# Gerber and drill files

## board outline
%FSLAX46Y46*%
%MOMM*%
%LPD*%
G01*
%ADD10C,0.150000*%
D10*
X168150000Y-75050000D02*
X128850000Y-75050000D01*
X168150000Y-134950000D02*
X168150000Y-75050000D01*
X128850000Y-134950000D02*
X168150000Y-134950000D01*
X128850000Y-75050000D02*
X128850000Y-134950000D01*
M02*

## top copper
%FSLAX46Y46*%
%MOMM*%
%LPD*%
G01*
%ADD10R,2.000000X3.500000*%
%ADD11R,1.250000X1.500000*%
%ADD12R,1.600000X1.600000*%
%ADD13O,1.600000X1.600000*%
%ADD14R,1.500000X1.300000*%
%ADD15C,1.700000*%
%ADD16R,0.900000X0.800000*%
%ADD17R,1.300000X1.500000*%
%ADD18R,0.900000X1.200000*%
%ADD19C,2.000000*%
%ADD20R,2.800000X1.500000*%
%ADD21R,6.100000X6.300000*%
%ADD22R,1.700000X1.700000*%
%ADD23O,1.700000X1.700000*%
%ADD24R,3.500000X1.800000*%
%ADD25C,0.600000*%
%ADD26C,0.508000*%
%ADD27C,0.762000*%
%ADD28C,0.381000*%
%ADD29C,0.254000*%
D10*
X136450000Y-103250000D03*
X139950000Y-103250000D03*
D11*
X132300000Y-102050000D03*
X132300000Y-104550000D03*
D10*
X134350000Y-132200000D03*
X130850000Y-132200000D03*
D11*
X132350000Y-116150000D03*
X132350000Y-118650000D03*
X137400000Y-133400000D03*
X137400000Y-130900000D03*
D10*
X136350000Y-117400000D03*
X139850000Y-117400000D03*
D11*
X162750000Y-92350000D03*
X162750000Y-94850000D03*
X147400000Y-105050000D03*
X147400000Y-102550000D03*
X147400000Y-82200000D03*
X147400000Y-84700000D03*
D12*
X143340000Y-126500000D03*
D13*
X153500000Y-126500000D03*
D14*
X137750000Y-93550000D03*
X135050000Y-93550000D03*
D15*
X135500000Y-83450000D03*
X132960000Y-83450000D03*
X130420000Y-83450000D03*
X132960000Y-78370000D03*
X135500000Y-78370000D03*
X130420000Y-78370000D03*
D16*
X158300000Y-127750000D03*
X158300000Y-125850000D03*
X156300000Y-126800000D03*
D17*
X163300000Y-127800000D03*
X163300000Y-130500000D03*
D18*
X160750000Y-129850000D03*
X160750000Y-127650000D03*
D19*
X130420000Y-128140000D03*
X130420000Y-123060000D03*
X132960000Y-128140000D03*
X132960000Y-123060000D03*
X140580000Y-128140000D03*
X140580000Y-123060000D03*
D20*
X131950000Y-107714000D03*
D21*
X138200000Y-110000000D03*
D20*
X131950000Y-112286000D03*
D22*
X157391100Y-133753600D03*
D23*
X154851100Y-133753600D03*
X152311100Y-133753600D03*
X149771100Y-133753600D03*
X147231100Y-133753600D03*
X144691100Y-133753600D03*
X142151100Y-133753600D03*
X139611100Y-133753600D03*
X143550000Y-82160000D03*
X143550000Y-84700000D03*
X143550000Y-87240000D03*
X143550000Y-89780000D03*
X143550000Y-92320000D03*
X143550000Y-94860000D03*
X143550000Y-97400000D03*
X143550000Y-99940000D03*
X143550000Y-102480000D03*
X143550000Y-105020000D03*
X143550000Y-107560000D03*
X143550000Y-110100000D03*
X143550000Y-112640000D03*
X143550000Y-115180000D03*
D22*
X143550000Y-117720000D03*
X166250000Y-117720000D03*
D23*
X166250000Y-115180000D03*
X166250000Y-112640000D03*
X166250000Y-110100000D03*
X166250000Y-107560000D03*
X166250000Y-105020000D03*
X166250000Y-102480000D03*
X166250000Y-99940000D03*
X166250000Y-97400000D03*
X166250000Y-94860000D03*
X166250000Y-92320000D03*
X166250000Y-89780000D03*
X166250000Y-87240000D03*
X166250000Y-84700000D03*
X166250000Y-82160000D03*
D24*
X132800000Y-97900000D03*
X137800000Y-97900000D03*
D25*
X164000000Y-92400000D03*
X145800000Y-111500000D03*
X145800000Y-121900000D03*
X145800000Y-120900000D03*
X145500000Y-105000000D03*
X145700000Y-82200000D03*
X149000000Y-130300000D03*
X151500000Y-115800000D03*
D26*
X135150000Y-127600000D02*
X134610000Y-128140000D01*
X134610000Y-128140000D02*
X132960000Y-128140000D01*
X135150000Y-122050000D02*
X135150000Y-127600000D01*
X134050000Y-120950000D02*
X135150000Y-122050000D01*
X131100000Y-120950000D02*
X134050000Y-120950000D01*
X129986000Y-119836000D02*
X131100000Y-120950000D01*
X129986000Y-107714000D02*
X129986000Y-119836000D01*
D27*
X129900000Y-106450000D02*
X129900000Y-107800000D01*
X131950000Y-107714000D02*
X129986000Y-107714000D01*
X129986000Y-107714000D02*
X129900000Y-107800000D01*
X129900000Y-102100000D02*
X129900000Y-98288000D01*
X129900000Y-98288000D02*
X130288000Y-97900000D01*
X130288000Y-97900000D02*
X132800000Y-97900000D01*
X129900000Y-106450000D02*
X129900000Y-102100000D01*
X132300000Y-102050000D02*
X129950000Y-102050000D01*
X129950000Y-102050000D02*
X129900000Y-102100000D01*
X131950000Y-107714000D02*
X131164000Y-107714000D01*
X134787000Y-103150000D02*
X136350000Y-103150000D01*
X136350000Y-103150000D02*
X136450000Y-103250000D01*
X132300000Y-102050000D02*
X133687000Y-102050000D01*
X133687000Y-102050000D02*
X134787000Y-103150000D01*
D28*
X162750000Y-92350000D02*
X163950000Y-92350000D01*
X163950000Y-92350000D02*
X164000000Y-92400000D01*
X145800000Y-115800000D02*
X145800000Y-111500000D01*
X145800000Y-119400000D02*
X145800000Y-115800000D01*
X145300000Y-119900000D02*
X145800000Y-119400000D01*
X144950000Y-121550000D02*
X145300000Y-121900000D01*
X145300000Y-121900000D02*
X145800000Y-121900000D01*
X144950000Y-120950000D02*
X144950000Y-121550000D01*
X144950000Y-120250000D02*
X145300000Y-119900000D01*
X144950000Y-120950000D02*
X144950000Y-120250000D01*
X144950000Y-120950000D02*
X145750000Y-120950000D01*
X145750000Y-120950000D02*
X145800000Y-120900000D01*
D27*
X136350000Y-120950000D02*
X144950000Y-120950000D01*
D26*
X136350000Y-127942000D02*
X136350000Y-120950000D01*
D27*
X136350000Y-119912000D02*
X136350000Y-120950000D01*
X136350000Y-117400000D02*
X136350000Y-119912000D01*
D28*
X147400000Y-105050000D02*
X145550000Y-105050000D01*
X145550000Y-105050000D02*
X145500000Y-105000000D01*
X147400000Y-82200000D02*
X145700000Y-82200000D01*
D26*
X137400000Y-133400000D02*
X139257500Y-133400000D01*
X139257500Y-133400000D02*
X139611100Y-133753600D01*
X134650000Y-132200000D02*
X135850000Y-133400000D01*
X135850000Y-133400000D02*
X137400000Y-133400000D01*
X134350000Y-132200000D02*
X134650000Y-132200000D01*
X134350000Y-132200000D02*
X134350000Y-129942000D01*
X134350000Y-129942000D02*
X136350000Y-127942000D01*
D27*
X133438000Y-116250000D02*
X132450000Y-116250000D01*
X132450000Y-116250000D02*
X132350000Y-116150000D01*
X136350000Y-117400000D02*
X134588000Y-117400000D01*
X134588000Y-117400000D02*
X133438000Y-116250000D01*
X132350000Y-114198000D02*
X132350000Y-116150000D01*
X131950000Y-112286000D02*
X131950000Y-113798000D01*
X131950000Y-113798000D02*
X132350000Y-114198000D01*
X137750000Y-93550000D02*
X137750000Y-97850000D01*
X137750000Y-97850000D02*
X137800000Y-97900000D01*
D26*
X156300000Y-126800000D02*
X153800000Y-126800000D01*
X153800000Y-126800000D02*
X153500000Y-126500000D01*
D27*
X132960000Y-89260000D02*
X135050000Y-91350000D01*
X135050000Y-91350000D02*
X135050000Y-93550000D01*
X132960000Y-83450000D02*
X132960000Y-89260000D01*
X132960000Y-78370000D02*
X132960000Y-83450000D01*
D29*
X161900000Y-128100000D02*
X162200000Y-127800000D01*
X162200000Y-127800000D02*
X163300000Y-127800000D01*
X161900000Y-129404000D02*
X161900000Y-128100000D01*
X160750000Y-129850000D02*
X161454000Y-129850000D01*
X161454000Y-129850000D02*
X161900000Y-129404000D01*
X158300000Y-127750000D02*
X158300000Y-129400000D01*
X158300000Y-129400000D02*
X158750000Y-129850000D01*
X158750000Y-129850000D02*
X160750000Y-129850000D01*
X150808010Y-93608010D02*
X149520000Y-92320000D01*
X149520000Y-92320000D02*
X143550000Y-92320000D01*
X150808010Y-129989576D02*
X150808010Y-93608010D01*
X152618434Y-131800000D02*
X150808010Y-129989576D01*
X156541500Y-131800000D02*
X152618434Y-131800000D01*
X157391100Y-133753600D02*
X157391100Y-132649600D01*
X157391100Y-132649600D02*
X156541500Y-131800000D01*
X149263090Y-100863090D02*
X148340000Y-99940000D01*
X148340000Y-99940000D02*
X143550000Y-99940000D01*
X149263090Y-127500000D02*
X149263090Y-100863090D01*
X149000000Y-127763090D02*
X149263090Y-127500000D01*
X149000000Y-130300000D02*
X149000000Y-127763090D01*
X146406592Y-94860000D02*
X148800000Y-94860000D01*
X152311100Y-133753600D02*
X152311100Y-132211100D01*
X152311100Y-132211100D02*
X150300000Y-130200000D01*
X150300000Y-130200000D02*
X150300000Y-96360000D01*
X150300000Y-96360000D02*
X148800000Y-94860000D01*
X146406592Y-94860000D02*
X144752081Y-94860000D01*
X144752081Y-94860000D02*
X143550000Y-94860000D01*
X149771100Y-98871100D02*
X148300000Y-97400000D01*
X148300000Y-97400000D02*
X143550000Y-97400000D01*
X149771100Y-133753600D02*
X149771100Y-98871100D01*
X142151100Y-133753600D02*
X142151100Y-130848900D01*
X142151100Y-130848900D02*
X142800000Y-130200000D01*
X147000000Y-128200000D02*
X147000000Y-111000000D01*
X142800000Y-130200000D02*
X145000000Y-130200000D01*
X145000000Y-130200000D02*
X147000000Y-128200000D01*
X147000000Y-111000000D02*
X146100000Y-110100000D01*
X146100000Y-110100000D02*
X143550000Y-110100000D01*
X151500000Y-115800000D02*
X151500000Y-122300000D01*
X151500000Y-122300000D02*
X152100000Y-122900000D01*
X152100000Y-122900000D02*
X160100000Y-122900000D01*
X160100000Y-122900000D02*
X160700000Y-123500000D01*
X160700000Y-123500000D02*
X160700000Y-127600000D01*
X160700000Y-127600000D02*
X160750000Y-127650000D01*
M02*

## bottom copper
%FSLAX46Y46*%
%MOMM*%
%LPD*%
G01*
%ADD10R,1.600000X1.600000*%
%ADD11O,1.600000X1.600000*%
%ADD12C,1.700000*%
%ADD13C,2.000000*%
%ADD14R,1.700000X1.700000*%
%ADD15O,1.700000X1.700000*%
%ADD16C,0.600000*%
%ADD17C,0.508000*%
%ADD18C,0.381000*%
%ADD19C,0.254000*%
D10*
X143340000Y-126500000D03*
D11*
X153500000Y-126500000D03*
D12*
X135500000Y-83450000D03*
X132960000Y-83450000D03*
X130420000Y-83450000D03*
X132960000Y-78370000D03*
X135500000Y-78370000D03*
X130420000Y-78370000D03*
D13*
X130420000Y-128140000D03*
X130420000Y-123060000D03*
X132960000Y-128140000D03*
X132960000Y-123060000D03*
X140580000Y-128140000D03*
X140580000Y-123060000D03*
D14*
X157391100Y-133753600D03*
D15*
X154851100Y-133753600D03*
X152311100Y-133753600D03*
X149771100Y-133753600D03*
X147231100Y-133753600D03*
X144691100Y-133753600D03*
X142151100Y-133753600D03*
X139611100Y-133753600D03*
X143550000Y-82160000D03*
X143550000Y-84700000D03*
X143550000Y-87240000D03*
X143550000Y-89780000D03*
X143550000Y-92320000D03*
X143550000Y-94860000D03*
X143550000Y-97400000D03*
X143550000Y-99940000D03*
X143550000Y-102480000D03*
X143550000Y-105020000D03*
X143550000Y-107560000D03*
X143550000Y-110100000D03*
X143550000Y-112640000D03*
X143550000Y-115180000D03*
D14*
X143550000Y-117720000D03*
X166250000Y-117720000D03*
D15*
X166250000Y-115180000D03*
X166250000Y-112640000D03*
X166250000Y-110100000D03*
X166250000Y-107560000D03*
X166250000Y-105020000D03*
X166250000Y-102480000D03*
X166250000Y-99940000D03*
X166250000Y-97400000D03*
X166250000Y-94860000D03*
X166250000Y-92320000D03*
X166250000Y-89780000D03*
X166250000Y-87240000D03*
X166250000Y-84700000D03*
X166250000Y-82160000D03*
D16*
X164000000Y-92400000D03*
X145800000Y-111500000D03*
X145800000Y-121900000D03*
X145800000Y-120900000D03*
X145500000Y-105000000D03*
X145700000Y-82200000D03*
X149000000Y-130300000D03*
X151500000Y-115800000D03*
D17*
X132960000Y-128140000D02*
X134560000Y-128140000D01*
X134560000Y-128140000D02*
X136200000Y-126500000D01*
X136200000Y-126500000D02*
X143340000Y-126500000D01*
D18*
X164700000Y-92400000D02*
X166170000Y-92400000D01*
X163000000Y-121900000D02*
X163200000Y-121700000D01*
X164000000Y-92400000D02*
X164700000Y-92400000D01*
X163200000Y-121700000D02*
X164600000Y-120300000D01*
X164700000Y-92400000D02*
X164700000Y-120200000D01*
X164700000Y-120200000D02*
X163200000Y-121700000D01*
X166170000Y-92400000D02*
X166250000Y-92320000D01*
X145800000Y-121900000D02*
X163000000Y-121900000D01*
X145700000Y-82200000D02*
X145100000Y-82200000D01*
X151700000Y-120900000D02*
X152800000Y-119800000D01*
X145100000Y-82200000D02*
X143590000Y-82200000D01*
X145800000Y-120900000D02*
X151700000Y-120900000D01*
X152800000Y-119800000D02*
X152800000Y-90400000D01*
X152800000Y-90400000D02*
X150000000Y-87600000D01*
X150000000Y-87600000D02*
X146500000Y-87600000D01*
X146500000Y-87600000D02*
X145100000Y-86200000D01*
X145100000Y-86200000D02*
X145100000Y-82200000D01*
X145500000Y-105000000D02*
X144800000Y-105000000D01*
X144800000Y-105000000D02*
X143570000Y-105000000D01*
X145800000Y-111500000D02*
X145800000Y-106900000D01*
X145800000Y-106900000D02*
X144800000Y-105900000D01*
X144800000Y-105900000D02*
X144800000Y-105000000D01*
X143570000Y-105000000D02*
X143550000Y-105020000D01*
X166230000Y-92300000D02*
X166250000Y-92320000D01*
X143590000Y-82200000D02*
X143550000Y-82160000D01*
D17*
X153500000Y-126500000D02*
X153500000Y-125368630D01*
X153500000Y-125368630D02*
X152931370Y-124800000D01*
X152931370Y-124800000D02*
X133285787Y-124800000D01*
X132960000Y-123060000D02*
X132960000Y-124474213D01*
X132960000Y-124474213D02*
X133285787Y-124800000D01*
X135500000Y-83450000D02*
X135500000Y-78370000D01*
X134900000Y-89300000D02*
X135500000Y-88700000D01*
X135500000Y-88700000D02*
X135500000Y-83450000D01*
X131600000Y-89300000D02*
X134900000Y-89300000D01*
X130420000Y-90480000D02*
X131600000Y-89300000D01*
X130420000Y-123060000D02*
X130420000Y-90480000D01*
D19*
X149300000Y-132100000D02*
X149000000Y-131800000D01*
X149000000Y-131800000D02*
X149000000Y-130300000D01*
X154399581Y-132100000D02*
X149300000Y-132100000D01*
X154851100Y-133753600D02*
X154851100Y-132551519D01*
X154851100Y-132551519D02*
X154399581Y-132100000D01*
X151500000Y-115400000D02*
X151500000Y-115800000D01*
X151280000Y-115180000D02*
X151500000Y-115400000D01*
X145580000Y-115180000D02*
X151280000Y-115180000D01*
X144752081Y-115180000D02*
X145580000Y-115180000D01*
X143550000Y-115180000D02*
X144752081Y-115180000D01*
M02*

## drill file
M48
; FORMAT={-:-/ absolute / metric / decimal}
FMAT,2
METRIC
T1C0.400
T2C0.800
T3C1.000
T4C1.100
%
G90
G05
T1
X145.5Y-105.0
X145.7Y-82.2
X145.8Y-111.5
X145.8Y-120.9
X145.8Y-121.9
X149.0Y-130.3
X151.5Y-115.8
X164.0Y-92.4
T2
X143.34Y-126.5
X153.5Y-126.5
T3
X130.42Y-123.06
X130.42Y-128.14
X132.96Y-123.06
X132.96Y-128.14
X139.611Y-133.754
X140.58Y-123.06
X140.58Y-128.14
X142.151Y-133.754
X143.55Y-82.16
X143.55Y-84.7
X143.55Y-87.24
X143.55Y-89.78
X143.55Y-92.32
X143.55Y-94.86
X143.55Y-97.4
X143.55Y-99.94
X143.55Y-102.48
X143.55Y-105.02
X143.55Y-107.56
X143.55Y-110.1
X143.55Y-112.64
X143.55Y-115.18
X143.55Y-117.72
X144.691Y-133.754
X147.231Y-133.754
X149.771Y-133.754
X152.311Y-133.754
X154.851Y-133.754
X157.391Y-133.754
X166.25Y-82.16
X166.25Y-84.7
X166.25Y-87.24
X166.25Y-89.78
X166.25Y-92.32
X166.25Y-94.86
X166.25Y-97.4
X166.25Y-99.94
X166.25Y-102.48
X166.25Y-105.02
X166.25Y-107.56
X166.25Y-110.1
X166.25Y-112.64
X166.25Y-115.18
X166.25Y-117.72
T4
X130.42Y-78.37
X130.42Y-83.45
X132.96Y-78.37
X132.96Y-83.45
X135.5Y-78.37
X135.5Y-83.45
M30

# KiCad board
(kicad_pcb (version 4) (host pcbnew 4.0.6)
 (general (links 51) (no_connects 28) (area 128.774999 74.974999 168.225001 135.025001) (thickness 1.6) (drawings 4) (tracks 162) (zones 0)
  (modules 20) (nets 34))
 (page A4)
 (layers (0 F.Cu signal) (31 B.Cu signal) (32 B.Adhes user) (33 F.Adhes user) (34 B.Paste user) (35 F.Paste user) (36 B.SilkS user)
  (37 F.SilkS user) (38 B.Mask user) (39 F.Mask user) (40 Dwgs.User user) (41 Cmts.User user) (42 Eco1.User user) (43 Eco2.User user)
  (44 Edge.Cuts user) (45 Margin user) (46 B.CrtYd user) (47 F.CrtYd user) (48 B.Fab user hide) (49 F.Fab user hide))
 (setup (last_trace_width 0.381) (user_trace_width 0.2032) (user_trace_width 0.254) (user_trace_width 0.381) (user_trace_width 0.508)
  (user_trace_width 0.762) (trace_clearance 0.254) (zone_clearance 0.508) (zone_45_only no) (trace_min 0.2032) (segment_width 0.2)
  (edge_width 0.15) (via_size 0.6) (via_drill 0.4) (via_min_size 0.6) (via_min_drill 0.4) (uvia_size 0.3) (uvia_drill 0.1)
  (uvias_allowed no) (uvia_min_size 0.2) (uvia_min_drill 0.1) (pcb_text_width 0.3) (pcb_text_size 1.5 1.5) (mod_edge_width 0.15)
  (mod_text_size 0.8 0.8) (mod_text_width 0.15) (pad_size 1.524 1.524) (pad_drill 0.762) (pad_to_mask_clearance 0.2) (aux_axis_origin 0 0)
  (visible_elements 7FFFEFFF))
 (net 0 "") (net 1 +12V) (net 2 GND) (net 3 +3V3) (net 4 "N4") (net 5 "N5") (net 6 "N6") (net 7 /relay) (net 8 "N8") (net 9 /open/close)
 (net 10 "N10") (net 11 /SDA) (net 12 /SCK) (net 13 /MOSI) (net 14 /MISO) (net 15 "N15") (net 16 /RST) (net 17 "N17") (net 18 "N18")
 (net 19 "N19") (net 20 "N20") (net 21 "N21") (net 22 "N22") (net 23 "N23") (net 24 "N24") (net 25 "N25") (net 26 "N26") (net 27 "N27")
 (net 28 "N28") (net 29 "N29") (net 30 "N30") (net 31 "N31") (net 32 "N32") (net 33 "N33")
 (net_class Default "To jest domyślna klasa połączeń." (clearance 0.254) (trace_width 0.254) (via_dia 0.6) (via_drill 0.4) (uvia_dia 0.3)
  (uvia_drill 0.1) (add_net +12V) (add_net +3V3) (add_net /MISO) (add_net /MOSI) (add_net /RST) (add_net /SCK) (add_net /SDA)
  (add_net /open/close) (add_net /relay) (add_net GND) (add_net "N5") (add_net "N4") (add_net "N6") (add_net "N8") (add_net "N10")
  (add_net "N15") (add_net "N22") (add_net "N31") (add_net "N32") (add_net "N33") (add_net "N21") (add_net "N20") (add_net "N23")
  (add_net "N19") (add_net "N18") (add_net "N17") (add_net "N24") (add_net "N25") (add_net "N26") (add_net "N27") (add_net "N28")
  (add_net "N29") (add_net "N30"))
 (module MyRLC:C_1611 (layer F.Cu) (at 138.2 103.25 90)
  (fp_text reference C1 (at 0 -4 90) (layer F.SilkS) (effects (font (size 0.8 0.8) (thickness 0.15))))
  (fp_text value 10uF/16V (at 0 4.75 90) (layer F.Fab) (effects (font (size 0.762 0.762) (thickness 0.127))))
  (pad 1 smd rect (at 0 -1.75 90) (size 3.5 2) (layers F.Cu F.Paste F.Mask) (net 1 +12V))
  (pad 2 smd rect (at 0 1.75 90) (size 3.5 2) (layers F.Cu F.Paste F.Mask) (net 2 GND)))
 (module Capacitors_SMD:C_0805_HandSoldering (layer F.Cu) (at 132.3 103.3 270)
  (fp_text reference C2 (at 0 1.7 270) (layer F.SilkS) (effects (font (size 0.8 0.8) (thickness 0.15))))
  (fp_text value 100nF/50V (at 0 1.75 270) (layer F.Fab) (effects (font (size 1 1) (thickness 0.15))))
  (pad 1 smd rect (at -1.25 0 270) (size 1.5 1.25) (layers F.Cu F.Paste F.Mask) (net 1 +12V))
  (pad 2 smd rect (at 1.25 0 270) (size 1.5 1.25) (layers F.Cu F.Paste F.Mask) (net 2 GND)))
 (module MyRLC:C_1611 (layer F.Cu) (at 132.6 132.2 270)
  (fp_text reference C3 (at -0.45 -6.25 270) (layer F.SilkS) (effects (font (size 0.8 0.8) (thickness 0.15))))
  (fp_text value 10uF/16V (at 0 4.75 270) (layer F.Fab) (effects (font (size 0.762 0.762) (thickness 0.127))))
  (pad 1 smd rect (at 0 -1.75 270) (size 3.5 2) (layers F.Cu F.Paste F.Mask) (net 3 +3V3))
  (pad 2 smd rect (at 0 1.75 270) (size 3.5 2) (layers F.Cu F.Paste F.Mask) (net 2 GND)))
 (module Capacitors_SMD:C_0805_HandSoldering (layer F.Cu) (at 132.35 117.4 270)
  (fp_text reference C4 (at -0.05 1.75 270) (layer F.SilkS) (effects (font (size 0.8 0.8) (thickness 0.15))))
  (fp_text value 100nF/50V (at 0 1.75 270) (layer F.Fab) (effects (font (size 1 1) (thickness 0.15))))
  (pad 1 smd rect (at -1.25 0 270) (size 1.5 1.25) (layers F.Cu F.Paste F.Mask) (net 3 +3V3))
  (pad 2 smd rect (at 1.25 0 270) (size 1.5 1.25) (layers F.Cu F.Paste F.Mask) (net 2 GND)))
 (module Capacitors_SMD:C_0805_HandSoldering (layer F.Cu) (at 137.4 132.15 90)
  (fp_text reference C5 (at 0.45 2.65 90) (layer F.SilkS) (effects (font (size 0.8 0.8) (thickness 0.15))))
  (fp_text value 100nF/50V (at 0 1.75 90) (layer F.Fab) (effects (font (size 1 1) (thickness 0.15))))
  (pad 1 smd rect (at -1.25 0 90) (size 1.5 1.25) (layers F.Cu F.Paste F.Mask) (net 3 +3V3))
  (pad 2 smd rect (at 1.25 0 90) (size 1.5 1.25) (layers F.Cu F.Paste F.Mask) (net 2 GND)))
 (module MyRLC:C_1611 (layer F.Cu) (at 138.1 117.4 90)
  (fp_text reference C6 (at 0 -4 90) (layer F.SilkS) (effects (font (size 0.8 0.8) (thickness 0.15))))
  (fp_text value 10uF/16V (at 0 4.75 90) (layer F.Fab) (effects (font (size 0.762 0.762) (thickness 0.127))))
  (pad 1 smd rect (at 0 -1.75 90) (size 3.5 2) (layers F.Cu F.Paste F.Mask) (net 3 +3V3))
  (pad 2 smd rect (at 0 1.75 90) (size 3.5 2) (layers F.Cu F.Paste F.Mask) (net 2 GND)))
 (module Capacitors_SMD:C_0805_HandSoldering (layer F.Cu) (at 162.75 93.6 270)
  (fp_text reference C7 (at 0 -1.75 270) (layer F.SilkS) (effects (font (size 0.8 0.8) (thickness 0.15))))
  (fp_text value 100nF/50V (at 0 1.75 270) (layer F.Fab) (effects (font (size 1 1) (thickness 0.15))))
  (pad 1 smd rect (at -1.25 0 270) (size 1.5 1.25) (layers F.Cu F.Paste F.Mask) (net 3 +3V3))
  (pad 2 smd rect (at 1.25 0 270) (size 1.5 1.25) (layers F.Cu F.Paste F.Mask) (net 2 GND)))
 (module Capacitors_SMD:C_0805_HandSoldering (layer F.Cu) (at 147.4 103.8 90)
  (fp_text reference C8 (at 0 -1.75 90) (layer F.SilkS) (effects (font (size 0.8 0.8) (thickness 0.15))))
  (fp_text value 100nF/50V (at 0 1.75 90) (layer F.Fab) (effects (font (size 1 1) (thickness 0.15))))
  (pad 1 smd rect (at -1.25 0 90) (size 1.5 1.25) (layers F.Cu F.Paste F.Mask) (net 3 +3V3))
  (pad 2 smd rect (at 1.25 0 90) (size 1.5 1.25) (layers F.Cu F.Paste F.Mask) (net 2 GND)))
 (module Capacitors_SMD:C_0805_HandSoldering (layer F.Cu) (at 147.4 83.45 270)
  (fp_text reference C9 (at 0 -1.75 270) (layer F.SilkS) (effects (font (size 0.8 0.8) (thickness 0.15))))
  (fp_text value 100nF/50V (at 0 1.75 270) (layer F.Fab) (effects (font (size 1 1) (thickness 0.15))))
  (pad 1 smd rect (at -1.25 0 270) (size 1.5 1.25) (layers F.Cu F.Paste F.Mask) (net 3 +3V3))
  (pad 2 smd rect (at 1.25 0 270) (size 1.5 1.25) (layers F.Cu F.Paste F.Mask) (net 2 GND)))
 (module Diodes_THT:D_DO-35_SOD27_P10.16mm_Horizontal (layer F.Cu) (at 143.34 126.5)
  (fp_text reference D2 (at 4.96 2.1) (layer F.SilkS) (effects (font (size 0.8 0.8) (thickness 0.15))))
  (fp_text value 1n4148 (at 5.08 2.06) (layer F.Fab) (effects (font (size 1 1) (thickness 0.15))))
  (pad 1 thru_hole rect (at 0 0) (size 1.6 1.6) (drill 0.8) (layers *.Cu *.Mask) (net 1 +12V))
  (pad 2 thru_hole oval (at 10.16 0) (size 1.6 1.6) (drill 0.8) (layers *.Cu *.Mask) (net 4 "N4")))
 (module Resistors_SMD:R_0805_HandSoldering (layer F.Cu) (at 136.4 93.55 180)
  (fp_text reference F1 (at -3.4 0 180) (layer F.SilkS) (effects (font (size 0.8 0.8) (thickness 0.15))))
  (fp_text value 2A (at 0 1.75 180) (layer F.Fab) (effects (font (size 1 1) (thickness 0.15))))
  (pad 1 smd rect (at -1.35 0 180) (size 1.5 1.3) (layers F.Cu F.Paste F.Mask) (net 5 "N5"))
  (pad 2 smd rect (at 1.35 0 180) (size 1.5 1.3) (layers F.Cu F.Paste F.Mask) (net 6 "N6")))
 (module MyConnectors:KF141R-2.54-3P (layer F.Cu) (at 132.96 80.91)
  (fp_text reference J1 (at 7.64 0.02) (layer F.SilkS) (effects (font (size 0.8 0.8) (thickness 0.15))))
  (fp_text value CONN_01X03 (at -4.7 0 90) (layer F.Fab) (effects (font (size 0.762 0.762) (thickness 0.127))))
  (pad 1 thru_hole circle (at 2.54 2.54) (size 1.7 1.7) (drill 1.1) (layers *.Cu *.Mask) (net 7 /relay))
  (pad 2 thru_hole circle (at 0 2.54) (size 1.7 1.7) (drill 1.1) (layers *.Cu *.Mask) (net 6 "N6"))
  (pad 3 thru_hole circle (at -2.54 2.54) (size 1.7 1.7) (drill 1.1) (layers *.Cu *.Mask) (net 2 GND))
  (pad 2 thru_hole circle (at 0 -2.54) (size 1.7 1.7) (drill 1.1) (layers *.Cu *.Mask) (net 6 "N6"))
  (pad 1 thru_hole circle (at 2.54 -2.54) (size 1.7 1.7) (drill 1.1) (layers *.Cu *.Mask) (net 7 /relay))
  (pad 3 thru_hole circle (at -2.54 -2.54) (size 1.7 1.7) (drill 1.1) (layers *.Cu *.Mask) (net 2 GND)))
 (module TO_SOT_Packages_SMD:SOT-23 (layer F.Cu) (at 157.3 126.8 180)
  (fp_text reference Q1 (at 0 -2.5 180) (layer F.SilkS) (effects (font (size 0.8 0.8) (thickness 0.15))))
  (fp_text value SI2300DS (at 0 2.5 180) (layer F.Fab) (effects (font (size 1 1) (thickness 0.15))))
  (pad 1 smd rect (at -1 -0.95 180) (size 0.9 0.8) (layers F.Cu F.Paste F.Mask) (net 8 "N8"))
  (pad 2 smd rect (at -1 0.95 180) (size 0.9 0.8) (layers F.Cu F.Paste F.Mask) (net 2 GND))
  (pad 3 smd rect (at 1 0 180) (size 0.9 0.8) (layers F.Cu F.Paste F.Mask) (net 4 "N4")))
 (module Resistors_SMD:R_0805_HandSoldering (layer F.Cu) (at 163.3 129.15 270)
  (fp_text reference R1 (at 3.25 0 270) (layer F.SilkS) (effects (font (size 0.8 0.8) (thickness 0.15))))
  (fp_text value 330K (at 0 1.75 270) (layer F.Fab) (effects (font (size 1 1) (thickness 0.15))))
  (pad 1 smd rect (at -1.35 0 270) (size 1.5 1.3) (layers F.Cu F.Paste F.Mask) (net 8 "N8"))
  (pad 2 smd rect (at 1.35 0 270) (size 1.5 1.3) (layers F.Cu F.Paste F.Mask) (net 2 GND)))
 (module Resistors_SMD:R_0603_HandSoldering (layer F.Cu) (at 160.75 128.75 90)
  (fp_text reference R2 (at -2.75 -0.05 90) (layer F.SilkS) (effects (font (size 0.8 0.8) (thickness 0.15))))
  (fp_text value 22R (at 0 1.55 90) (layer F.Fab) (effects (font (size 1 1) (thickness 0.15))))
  (pad 1 smd rect (at -1.1 0 90) (size 1.2 0.9) (layers F.Cu F.Paste F.Mask) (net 8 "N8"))
  (pad 2 smd rect (at 1.1 0 90) (size 1.2 0.9) (layers F.Cu F.Paste F.Mask) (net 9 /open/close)))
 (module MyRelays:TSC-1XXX (layer F.Cu) (at 135.5 125.6 90)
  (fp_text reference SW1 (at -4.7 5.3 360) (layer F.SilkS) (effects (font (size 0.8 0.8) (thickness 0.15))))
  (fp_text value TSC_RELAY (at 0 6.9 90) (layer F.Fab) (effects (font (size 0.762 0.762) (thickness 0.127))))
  (pad 1 thru_hole circle (at -2.54 -5.08 90) (size 2 2) (drill 1) (layers *.Cu *.Mask) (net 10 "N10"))
  (pad 2 thru_hole circle (at 2.54 -5.08 90) (size 2 2) (drill 1) (layers *.Cu *.Mask) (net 7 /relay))
  (pad 3 thru_hole circle (at -2.54 -2.54 90) (size 2 2) (drill 1) (layers *.Cu *.Mask) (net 1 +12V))
  (pad 4 thru_hole circle (at 2.54 -2.54 90) (size 2 2) (drill 1) (layers *.Cu *.Mask) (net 4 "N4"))
  (pad 5 thru_hole circle (at -2.54 5.08 90) (size 2 2) (drill 1) (layers *.Cu *.Mask) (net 2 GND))
  (pad 6 thru_hole circle (at 2.54 5.08 90) (size 2 2) (drill 1) (layers *.Cu *.Mask) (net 2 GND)))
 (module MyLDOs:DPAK (layer F.Cu) (at 135.9 110 270)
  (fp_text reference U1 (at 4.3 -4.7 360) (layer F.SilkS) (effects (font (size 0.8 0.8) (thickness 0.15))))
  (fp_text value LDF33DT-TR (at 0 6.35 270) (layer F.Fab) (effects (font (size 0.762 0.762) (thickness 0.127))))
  (pad 1 smd rect (at -2.286 3.95 270) (size 1.5 2.8) (layers F.Cu F.Paste F.Mask) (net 1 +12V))
  (pad 2 smd rect (at 0 -2.3 270) (size 6.3 6.1) (layers F.Cu F.Paste F.Mask) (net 2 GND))
  (pad 3 smd rect (at 2.286 3.95 270) (size 1.5 2.8) (layers F.Cu F.Paste F.Mask) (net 3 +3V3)))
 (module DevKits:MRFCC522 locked (layer B.Cu) (at 148.5011 105.0036)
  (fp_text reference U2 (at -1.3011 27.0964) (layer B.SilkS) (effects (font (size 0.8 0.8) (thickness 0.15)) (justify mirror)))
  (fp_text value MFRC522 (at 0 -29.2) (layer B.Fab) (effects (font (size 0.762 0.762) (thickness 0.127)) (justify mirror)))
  (pad 1 thru_hole rect (at 8.89 28.75 90) (size 1.7 1.7) (drill 1) (layers *.Cu *.Mask) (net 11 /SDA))
  (pad 2 thru_hole oval (at 6.35 28.75 90) (size 1.7 1.7) (drill 1) (layers *.Cu *.Mask) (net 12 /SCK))
  (pad 3 thru_hole oval (at 3.81 28.75 90) (size 1.7 1.7) (drill 1) (layers *.Cu *.Mask) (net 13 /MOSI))
  (pad 4 thru_hole oval (at 1.27 28.75 90) (size 1.7 1.7) (drill 1) (layers *.Cu *.Mask) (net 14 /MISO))
  (pad 5 thru_hole oval (at -1.27 28.75 90) (size 1.7 1.7) (drill 1) (layers *.Cu *.Mask) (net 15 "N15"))
  (pad 6 thru_hole oval (at -3.81 28.75 90) (size 1.7 1.7) (drill 1) (layers *.Cu *.Mask) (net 2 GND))
  (pad 7 thru_hole oval (at -6.35 28.75 90) (size 1.7 1.7) (drill 1) (layers *.Cu *.Mask) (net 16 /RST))
  (pad 8 thru_hole oval (at -8.89 28.75 90) (size 1.7 1.7) (drill 1) (layers *.Cu *.Mask) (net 3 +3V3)))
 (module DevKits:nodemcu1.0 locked (layer F.Cu) (at 154.9 99.94 180)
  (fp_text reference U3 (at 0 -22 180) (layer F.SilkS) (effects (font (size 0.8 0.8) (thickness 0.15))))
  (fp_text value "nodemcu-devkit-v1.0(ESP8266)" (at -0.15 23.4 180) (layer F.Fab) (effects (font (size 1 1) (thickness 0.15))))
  (pad 30 thru_hole oval (at 11.35 17.78 180) (size 1.7 1.7) (drill 1) (layers *.Cu *.Mask) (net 3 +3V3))
  (pad 29 thru_hole oval (at 11.35 15.24 180) (size 1.7 1.7) (drill 1) (layers *.Cu *.Mask) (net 2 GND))
  (pad 28 thru_hole oval (at 11.35 12.7 180) (size 1.7 1.7) (drill 1) (layers *.Cu *.Mask) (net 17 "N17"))
  (pad 27 thru_hole oval (at 11.35 10.16 180) (size 1.7 1.7) (drill 1) (layers *.Cu *.Mask) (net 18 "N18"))
  (pad 26 thru_hole oval (at 11.35 7.62 180) (size 1.7 1.7) (drill 1) (layers *.Cu *.Mask) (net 11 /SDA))
  (pad 25 thru_hole oval (at 11.35 5.08 180) (size 1.7 1.7) (drill 1) (layers *.Cu *.Mask) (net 13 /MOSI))
  (pad 24 thru_hole oval (at 11.35 2.54 180) (size 1.7 1.7) (drill 1) (layers *.Cu *.Mask) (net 14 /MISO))
  (pad 23 thru_hole oval (at 11.35 0 180) (size 1.7 1.7) (drill 1) (layers *.Cu *.Mask) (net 12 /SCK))
  (pad 22 thru_hole oval (at 11.35 -2.54 180) (size 1.7 1.7) (drill 1) (layers *.Cu *.Mask) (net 2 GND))
  (pad 21 thru_hole oval (at 11.35 -5.08 180) (size 1.7 1.7) (drill 1) (layers *.Cu *.Mask) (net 3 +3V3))
  (pad 20 thru_hole oval (at 11.35 -7.62 180) (size 1.7 1.7) (drill 1) (layers *.Cu *.Mask) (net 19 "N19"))
  (pad 19 thru_hole oval (at 11.35 -10.16 180) (size 1.7 1.7) (drill 1) (layers *.Cu *.Mask) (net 16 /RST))
  (pad 18 thru_hole oval (at 11.35 -12.7 180) (size 1.7 1.7) (drill 1) (layers *.Cu *.Mask) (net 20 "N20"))
  (pad 17 thru_hole oval (at 11.35 -15.24 180) (size 1.7 1.7) (drill 1) (layers *.Cu *.Mask) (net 9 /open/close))
  (pad 16 thru_hole rect (at 11.35 -17.78 180) (size 1.7 1.7) (drill 1) (layers *.Cu *.Mask) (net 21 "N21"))
  (pad 1 thru_hole rect (at -11.35 -17.78 180) (size 1.7 1.7) (drill 1) (layers *.Cu *.Mask) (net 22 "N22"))
  (pad 2 thru_hole oval (at -11.35 -15.24 180) (size 1.7 1.7) (drill 1) (layers *.Cu *.Mask) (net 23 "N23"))
  (pad 3 thru_hole oval (at -11.35 -12.7 180) (size 1.7 1.7) (drill 1) (layers *.Cu *.Mask) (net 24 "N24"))
  (pad 4 thru_hole oval (at -11.35 -10.16 180) (size 1.7 1.7) (drill 1) (layers *.Cu *.Mask) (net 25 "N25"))
  (pad 5 thru_hole oval (at -11.35 -7.62 180) (size 1.7 1.7) (drill 1) (layers *.Cu *.Mask) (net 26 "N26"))
  (pad 6 thru_hole oval (at -11.35 -5.08 180) (size 1.7 1.7) (drill 1) (layers *.Cu *.Mask) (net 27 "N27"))
  (pad 7 thru_hole oval (at -11.35 -2.54 180) (size 1.7 1.7) (drill 1) (layers *.Cu *.Mask) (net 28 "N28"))
  (pad 8 thru_hole oval (at -11.35 0 180) (size 1.7 1.7) (drill 1) (layers *.Cu *.Mask) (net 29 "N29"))
  (pad 9 thru_hole oval (at -11.35 2.54 180) (size 1.7 1.7) (drill 1) (layers *.Cu *.Mask) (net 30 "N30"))
  (pad 10 thru_hole oval (at -11.35 5.08 180) (size 1.7 1.7) (drill 1) (layers *.Cu *.Mask) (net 2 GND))
  (pad 11 thru_hole oval (at -11.35 7.62 180) (size 1.7 1.7) (drill 1) (layers *.Cu *.Mask) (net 3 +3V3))
  (pad 12 thru_hole oval (at -11.35 10.16 180) (size 1.7 1.7) (drill 1) (layers *.Cu *.Mask) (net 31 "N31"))
  (pad 13 thru_hole oval (at -11.35 12.7 180) (size 1.7 1.7) (drill 1) (layers *.Cu *.Mask) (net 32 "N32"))
  (pad 14 thru_hole oval (at -11.35 15.24 180) (size 1.7 1.7) (drill 1) (layers *.Cu *.Mask) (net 2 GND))
  (pad 15 thru_hole oval (at -11.35 17.78 180) (size 1.7 1.7) (drill 1) (layers *.Cu *.Mask) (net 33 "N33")))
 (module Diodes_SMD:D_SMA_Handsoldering (layer F.Cu) (at 135.3 97.9)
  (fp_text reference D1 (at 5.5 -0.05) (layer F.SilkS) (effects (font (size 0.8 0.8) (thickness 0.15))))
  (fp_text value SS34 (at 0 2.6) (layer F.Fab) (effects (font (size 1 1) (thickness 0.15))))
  (pad 1 smd rect (at -2.5 0) (size 3.5 1.8) (layers F.Cu F.Paste F.Mask) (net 1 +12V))
  (pad 2 smd rect (at 2.5 0) (size 3.5 1.8) (layers F.Cu F.Paste F.Mask) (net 5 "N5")))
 (gr_line (start 168.15 75.05) (end 128.85 75.05) (layer Edge.Cuts) (width 0.15))
 (gr_line (start 168.15 134.95) (end 168.15 75.05) (layer Edge.Cuts) (width 0.15))
 (gr_line (start 128.85 134.95) (end 168.15 134.95) (layer Edge.Cuts) (width 0.15))
 (gr_line (start 128.85 75.05) (end 128.85 134.95) (layer Edge.Cuts) (width 0.15))
 (segment (start 132.96 128.14) (end 134.56 128.14) (width 0.508) (layer B.Cu) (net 1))
 (segment (start 134.56 128.14) (end 136.2 126.5) (width 0.508) (layer B.Cu) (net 1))
 (segment (start 136.2 126.5) (end 143.34 126.5) (width 0.508) (layer B.Cu) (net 1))
 (segment (start 135.15 127.6) (end 134.61 128.14) (width 0.508) (layer F.Cu) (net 1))
 (segment (start 134.61 128.14) (end 132.96 128.14) (width 0.508) (layer F.Cu) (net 1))
 (segment (start 135.15 122.05) (end 135.15 127.6) (width 0.508) (layer F.Cu) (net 1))
 (segment (start 134.05 120.95) (end 135.15 122.05) (width 0.508) (layer F.Cu) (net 1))
 (segment (start 131.1 120.95) (end 134.05 120.95) (width 0.508) (layer F.Cu) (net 1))
 (segment (start 129.986 119.836) (end 131.1 120.95) (width 0.508) (layer F.Cu) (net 1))
 (segment (start 129.986 107.714) (end 129.986 119.836) (width 0.508) (layer F.Cu) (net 1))
 (segment (start 129.9 106.45) (end 129.9 107.8) (width 0.762) (layer F.Cu) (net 1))
 (segment (start 131.95 107.714) (end 129.986 107.714) (width 0.762) (layer F.Cu) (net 1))
 (segment (start 129.986 107.714) (end 129.9 107.8) (width 0.762) (layer F.Cu) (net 1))
 (segment (start 129.9 102.1) (end 129.9 98.288) (width 0.762) (layer F.Cu) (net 1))
 (segment (start 129.9 98.288) (end 130.288 97.9) (width 0.762) (layer F.Cu) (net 1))
 (segment (start 130.288 97.9) (end 132.8 97.9) (width 0.762) (layer F.Cu) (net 1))
 (segment (start 129.9 106.45) (end 129.9 102.1) (width 0.762) (layer F.Cu) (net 1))
 (segment (start 132.3 102.05) (end 129.95 102.05) (width 0.762) (layer F.Cu) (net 1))
 (segment (start 129.95 102.05) (end 129.9 102.1) (width 0.762) (layer F.Cu) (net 1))
 (segment (start 131.95 107.714) (end 131.164 107.714) (width 0.762) (layer F.Cu) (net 1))
 (segment (start 134.787 103.15) (end 136.35 103.15) (width 0.762) (layer F.Cu) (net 1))
 (segment (start 136.35 103.15) (end 136.45 103.25) (width 0.762) (layer F.Cu) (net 1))
 (segment (start 132.3 102.05) (end 133.687 102.05) (width 0.762) (layer F.Cu) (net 1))
 (segment (start 133.687 102.05) (end 134.787 103.15) (width 0.762) (layer F.Cu) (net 1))
 (segment (start 164.7 92.4) (end 166.17 92.4) (width 0.381) (layer B.Cu) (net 3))
 (segment (start 163 121.9) (end 163.2 121.7) (width 0.381) (layer B.Cu) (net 3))
 (segment (start 164 92.4) (end 164.7 92.4) (width 0.381) (layer B.Cu) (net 3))
 (segment (start 163.2 121.7) (end 164.6 120.3) (width 0.381) (layer B.Cu) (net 3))
 (segment (start 164.7 92.4) (end 164.7 120.2) (width 0.381) (layer B.Cu) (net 3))
 (segment (start 164.7 120.2) (end 163.2 121.7) (width 0.381) (layer B.Cu) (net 3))
 (segment (start 166.17 92.4) (end 166.25 92.32) (width 0.381) (layer B.Cu) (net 3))
 (segment (start 162.75 92.35) (end 163.95 92.35) (width 0.381) (layer F.Cu) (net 3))
 (segment (start 163.95 92.35) (end 164 92.4) (width 0.381) (layer F.Cu) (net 3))
 (via (at 164 92.4) (size 0.6) (drill 0.4) (layers F.Cu B.Cu) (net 3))
 (segment (start 145.8 121.9) (end 163 121.9) (width 0.381) (layer B.Cu) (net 3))
 (segment (start 145.7 82.2) (end 145.1 82.2) (width 0.381) (layer B.Cu) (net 3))
 (segment (start 151.7 120.9) (end 152.8 119.8) (width 0.381) (layer B.Cu) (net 3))
 (segment (start 145.1 82.2) (end 143.59 82.2) (width 0.381) (layer B.Cu) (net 3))
 (segment (start 145.8 120.9) (end 151.7 120.9) (width 0.381) (layer B.Cu) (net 3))
 (segment (start 152.8 119.8) (end 152.8 90.4) (width 0.381) (layer B.Cu) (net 3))
 (segment (start 152.8 90.4) (end 150 87.6) (width 0.381) (layer B.Cu) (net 3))
 (segment (start 150 87.6) (end 146.5 87.6) (width 0.381) (layer B.Cu) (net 3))
 (segment (start 146.5 87.6) (end 145.1 86.2) (width 0.381) (layer B.Cu) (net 3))
 (segment (start 145.1 86.2) (end 145.1 82.2) (width 0.381) (layer B.Cu) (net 3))
 (segment (start 145.5 105) (end 144.8 105) (width 0.381) (layer B.Cu) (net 3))
 (segment (start 144.8 105) (end 143.57 105) (width 0.381) (layer B.Cu) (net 3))
 (segment (start 145.8 111.5) (end 145.8 106.9) (width 0.381) (layer B.Cu) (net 3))
 (segment (start 145.8 106.9) (end 144.8 105.9) (width 0.381) (layer B.Cu) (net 3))
 (segment (start 144.8 105.9) (end 144.8 105) (width 0.381) (layer B.Cu) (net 3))
 (via (at 145.8 111.5) (size 0.6) (drill 0.4) (layers F.Cu B.Cu) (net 3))
 (segment (start 145.8 115.8) (end 145.8 111.5) (width 0.381) (layer F.Cu) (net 3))
 (segment (start 145.8 119.4) (end 145.8 115.8) (width 0.381) (layer F.Cu) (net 3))
 (segment (start 145.3 119.9) (end 145.8 119.4) (width 0.381) (layer F.Cu) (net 3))
 (segment (start 144.95 121.55) (end 145.3 121.9) (width 0.381) (layer F.Cu) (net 3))
 (segment (start 145.3 121.9) (end 145.8 121.9) (width 0.381) (layer F.Cu) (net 3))
 (via (at 145.8 121.9) (size 0.6) (drill 0.4) (layers F.Cu B.Cu) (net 3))
 (segment (start 144.95 120.95) (end 144.95 121.55) (width 0.381) (layer F.Cu) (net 3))
 (segment (start 144.95 120.25) (end 145.3 119.9) (width 0.381) (layer F.Cu) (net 3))
 (segment (start 144.95 120.95) (end 144.95 120.25) (width 0.381) (layer F.Cu) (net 3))
 (segment (start 144.95 120.95) (end 145.75 120.95) (width 0.381) (layer F.Cu) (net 3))
 (segment (start 145.75 120.95) (end 145.8 120.9) (width 0.381) (layer F.Cu) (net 3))
 (via (at 145.8 120.9) (size 0.6) (drill 0.4) (layers F.Cu B.Cu) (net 3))
 (segment (start 136.35 120.95) (end 144.95 120.95) (width 0.762) (layer F.Cu) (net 3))
 (segment (start 136.35 127.942) (end 136.35 120.95) (width 0.508) (layer F.Cu) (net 3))
 (segment (start 136.35 119.912) (end 136.35 120.95) (width 0.762) (layer F.Cu) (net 3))
 (segment (start 136.35 117.4) (end 136.35 119.912) (width 0.762) (layer F.Cu) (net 3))
 (segment (start 143.57 105) (end 143.55 105.02) (width 0.381) (layer B.Cu) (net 3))
 (segment (start 147.4 105.05) (end 145.55 105.05) (width 0.381) (layer F.Cu) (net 3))
 (segment (start 145.55 105.05) (end 145.5 105) (width 0.381) (layer F.Cu) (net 3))
 (via (at 145.5 105) (size 0.6) (drill 0.4) (layers F.Cu B.Cu) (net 3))
 (segment (start 166.23 92.3) (end 166.25 92.32) (width 0.381) (layer B.Cu) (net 3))
 (segment (start 143.59 82.2) (end 143.55 82.16) (width 0.381) (layer B.Cu) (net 3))
 (segment (start 147.4 82.2) (end 145.7 82.2) (width 0.381) (layer F.Cu) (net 3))
 (via (at 145.7 82.2) (size 0.6) (drill 0.4) (layers F.Cu B.Cu) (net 3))
 (segment (start 137.4 133.4) (end 139.2575 133.4) (width 0.508) (layer F.Cu) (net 3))
 (segment (start 139.2575 133.4) (end 139.6111 133.7536) (width 0.508) (layer F.Cu) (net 3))
 (segment (start 134.65 132.2) (end 135.85 133.4) (width 0.508) (layer F.Cu) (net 3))
 (segment (start 135.85 133.4) (end 137.4 133.4) (width 0.508) (layer F.Cu) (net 3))
 (segment (start 134.35 132.2) (end 134.65 132.2) (width 0.508) (layer F.Cu) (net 3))
 (segment (start 134.35 132.2) (end 134.35 129.942) (width 0.508) (layer F.Cu) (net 3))
 (segment (start 134.35 129.942) (end 136.35 127.942) (width 0.508) (layer F.Cu) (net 3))
 (segment (start 133.438 116.25) (end 132.45 116.25) (width 0.762) (layer F.Cu) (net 3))
 (segment (start 132.45 116.25) (end 132.35 116.15) (width 0.762) (layer F.Cu) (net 3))
 (segment (start 136.35 117.4) (end 134.588 117.4) (width 0.762) (layer F.Cu) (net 3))
 (segment (start 134.588 117.4) (end 133.438 116.25) (width 0.762) (layer F.Cu) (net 3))
 (segment (start 132.35 114.198) (end 132.35 116.15) (width 0.762) (layer F.Cu) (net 3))
 (segment (start 131.95 112.286) (end 131.95 113.798) (width 0.762) (layer F.Cu) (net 3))
 (segment (start 131.95 113.798) (end 132.35 114.198) (width 0.762) (layer F.Cu) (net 3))
 (segment (start 137.75 93.55) (end 137.75 97.85) (width 0.762) (layer F.Cu) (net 5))
 (segment (start 137.75 97.85) (end 137.8 97.9) (width 0.762) (layer F.Cu) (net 5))
 (segment (start 156.3 126.8) (end 153.8 126.8) (width 0.508) (layer F.Cu) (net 4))
 (segment (start 153.8 126.8) (end 153.5 126.5) (width 0.508) (layer F.Cu) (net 4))
 (segment (start 153.5 126.5) (end 153.5 125.36863) (width 0.508) (layer B.Cu) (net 4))
 (segment (start 153.5 125.36863) (end 152.93137 124.8) (width 0.508) (layer B.Cu) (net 4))
 (segment (start 152.93137 124.8) (end 133.285787 124.8) (width 0.508) (layer B.Cu) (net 4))
 (segment (start 132.96 123.06) (end 132.96 124.474213) (width 0.508) (layer B.Cu) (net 4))
 (segment (start 132.96 124.474213) (end 133.285787 124.8) (width 0.508) (layer B.Cu) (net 4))
 (segment (start 132.96 89.26) (end 135.05 91.35) (width 0.762) (layer F.Cu) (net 6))
 (segment (start 135.05 91.35) (end 135.05 93.55) (width 0.762) (layer F.Cu) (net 6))
 (segment (start 132.96 83.45) (end 132.96 89.26) (width 0.762) (layer F.Cu) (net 6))
 (segment (start 132.96 78.37) (end 132.96 83.45) (width 0.762) (layer F.Cu) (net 6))
 (segment (start 135.5 83.45) (end 135.5 78.37) (width 0.508) (layer B.Cu) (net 7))
 (segment (start 134.9 89.3) (end 135.5 88.7) (width 0.508) (layer B.Cu) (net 7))
 (segment (start 135.5 88.7) (end 135.5 83.45) (width 0.508) (layer B.Cu) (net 7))
 (segment (start 131.6 89.3) (end 134.9 89.3) (width 0.508) (layer B.Cu) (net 7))
 (segment (start 130.42 90.48) (end 131.6 89.3) (width 0.508) (layer B.Cu) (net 7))
 (segment (start 130.42 123.06) (end 130.42 90.48) (width 0.508) (layer B.Cu) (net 7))
 (segment (start 161.9 128.1) (end 162.2 127.8) (width 0.254) (layer F.Cu) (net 8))
 (segment (start 162.2 127.8) (end 163.3 127.8) (width 0.254) (layer F.Cu) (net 8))
 (segment (start 161.9 129.404) (end 161.9 128.1) (width 0.254) (layer F.Cu) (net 8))
 (segment (start 160.75 129.85) (end 161.454 129.85) (width 0.254) (layer F.Cu) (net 8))
 (segment (start 161.454 129.85) (end 161.9 129.404) (width 0.254) (layer F.Cu) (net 8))
 (segment (start 158.3 127.75) (end 158.3 129.4) (width 0.254) (layer F.Cu) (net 8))
 (segment (start 158.3 129.4) (end 158.75 129.85) (width 0.254) (layer F.Cu) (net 8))
 (segment (start 158.75 129.85) (end 160.75 129.85) (width 0.254) (layer F.Cu) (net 8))
 (segment (start 150.80801 93.60801) (end 149.52 92.32) (width 0.254) (layer F.Cu) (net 11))
 (segment (start 149.52 92.32) (end 143.55 92.32) (width 0.254) (layer F.Cu) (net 11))
 (segment (start 150.80801 129.989576) (end 150.80801 93.60801) (width 0.254) (layer F.Cu) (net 11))
 (segment (start 152.618434 131.8) (end 150.80801 129.989576) (width 0.254) (layer F.Cu) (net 11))
 (segment (start 156.5415 131.8) (end 152.618434 131.8) (width 0.254) (layer F.Cu) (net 11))
 (segment (start 157.3911 133.7536) (end 157.3911 132.6496) (width 0.254) (layer F.Cu) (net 11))
 (segment (start 157.3911 132.6496) (end 156.5415 131.8) (width 0.254) (layer F.Cu) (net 11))
 (segment (start 149.26309 100.86309) (end 148.34 99.94) (width 0.254) (layer F.Cu) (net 12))
 (segment (start 148.34 99.94) (end 143.55 99.94) (width 0.254) (layer F.Cu) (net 12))
 (segment (start 149.26309 127.5) (end 149.26309 100.86309) (width 0.254) (layer F.Cu) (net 12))
 (segment (start 149 127.76309) (end 149.26309 127.5) (width 0.254) (layer F.Cu) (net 12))
 (segment (start 149 130.3) (end 149 127.76309) (width 0.254) (layer F.Cu) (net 12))
 (segment (start 149.3 132.1) (end 149 131.8) (width 0.254) (layer B.Cu) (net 12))
 (segment (start 149 131.8) (end 149 130.3) (width 0.254) (layer B.Cu) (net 12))
 (via (at 149 130.3) (size 0.6) (drill 0.4) (layers F.Cu B.Cu) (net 12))
 (segment (start 154.399581 132.1) (end 149.3 132.1) (width 0.254) (layer B.Cu) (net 12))
 (segment (start 154.8511 133.7536) (end 154.8511 132.551519) (width 0.254) (layer B.Cu) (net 12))
 (segment (start 154.8511 132.551519) (end 154.399581 132.1) (width 0.254) (layer B.Cu) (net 12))
 (segment (start 146.406592 94.86) (end 148.8 94.86) (width 0.254) (layer F.Cu) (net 13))
 (segment (start 152.3111 133.7536) (end 152.3111 132.2111) (width 0.254) (layer F.Cu) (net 13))
 (segment (start 152.3111 132.2111) (end 150.3 130.2) (width 0.254) (layer F.Cu) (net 13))
 (segment (start 150.3 130.2) (end 150.3 96.36) (width 0.254) (layer F.Cu) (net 13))
 (segment (start 150.3 96.36) (end 148.8 94.86) (width 0.254) (layer F.Cu) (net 13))
 (segment (start 146.406592 94.86) (end 144.752081 94.86) (width 0.254) (layer F.Cu) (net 13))
 (segment (start 144.752081 94.86) (end 143.55 94.86) (width 0.254) (layer F.Cu) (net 13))
 (segment (start 149.7711 98.8711) (end 148.3 97.4) (width 0.254) (layer F.Cu) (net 14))
 (segment (start 148.3 97.4) (end 143.55 97.4) (width 0.254) (layer F.Cu) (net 14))
 (segment (start 149.7711 133.7536) (end 149.7711 98.8711) (width 0.254) (layer F.Cu) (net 14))
 (segment (start 142.1511 133.7536) (end 142.1511 130.8489) (width 0.254) (layer F.Cu) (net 16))
 (segment (start 142.1511 130.8489) (end 142.8 130.2) (width 0.254) (layer F.Cu) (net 16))
 (segment (start 147 128.2) (end 147 111) (width 0.254) (layer F.Cu) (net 16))
 (segment (start 142.8 130.2) (end 145 130.2) (width 0.254) (layer F.Cu) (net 16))
 (segment (start 145 130.2) (end 147 128.2) (width 0.254) (layer F.Cu) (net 16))
 (segment (start 147 111) (end 146.1 110.1) (width 0.254) (layer F.Cu) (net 16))
 (segment (start 146.1 110.1) (end 143.55 110.1) (width 0.254) (layer F.Cu) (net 16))
 (segment (start 151.5 115.8) (end 151.5 122.3) (width 0.254) (layer F.Cu) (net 9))
 (segment (start 151.5 122.3) (end 152.1 122.9) (width 0.254) (layer F.Cu) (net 9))
 (segment (start 152.1 122.9) (end 160.1 122.9) (width 0.254) (layer F.Cu) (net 9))
 (segment (start 160.1 122.9) (end 160.7 123.5) (width 0.254) (layer F.Cu) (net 9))
 (segment (start 160.7 123.5) (end 160.7 127.6) (width 0.254) (layer F.Cu) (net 9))
 (segment (start 160.7 127.6) (end 160.75 127.65) (width 0.254) (layer F.Cu) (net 9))
 (segment (start 151.5 115.4) (end 151.5 115.8) (width 0.254) (layer B.Cu) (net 9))
 (via (at 151.5 115.8) (size 0.6) (drill 0.4) (layers F.Cu B.Cu) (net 9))
 (segment (start 151.28 115.18) (end 151.5 115.4) (width 0.254) (layer B.Cu) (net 9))
 (segment (start 145.58 115.18) (end 151.28 115.18) (width 0.254) (layer B.Cu) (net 9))
 (segment (start 144.752081 115.18) (end 145.58 115.18) (width 0.254) (layer B.Cu) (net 9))
 (segment (start 143.55 115.18) (end 144.752081 115.18) (width 0.254) (layer B.Cu) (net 9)))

